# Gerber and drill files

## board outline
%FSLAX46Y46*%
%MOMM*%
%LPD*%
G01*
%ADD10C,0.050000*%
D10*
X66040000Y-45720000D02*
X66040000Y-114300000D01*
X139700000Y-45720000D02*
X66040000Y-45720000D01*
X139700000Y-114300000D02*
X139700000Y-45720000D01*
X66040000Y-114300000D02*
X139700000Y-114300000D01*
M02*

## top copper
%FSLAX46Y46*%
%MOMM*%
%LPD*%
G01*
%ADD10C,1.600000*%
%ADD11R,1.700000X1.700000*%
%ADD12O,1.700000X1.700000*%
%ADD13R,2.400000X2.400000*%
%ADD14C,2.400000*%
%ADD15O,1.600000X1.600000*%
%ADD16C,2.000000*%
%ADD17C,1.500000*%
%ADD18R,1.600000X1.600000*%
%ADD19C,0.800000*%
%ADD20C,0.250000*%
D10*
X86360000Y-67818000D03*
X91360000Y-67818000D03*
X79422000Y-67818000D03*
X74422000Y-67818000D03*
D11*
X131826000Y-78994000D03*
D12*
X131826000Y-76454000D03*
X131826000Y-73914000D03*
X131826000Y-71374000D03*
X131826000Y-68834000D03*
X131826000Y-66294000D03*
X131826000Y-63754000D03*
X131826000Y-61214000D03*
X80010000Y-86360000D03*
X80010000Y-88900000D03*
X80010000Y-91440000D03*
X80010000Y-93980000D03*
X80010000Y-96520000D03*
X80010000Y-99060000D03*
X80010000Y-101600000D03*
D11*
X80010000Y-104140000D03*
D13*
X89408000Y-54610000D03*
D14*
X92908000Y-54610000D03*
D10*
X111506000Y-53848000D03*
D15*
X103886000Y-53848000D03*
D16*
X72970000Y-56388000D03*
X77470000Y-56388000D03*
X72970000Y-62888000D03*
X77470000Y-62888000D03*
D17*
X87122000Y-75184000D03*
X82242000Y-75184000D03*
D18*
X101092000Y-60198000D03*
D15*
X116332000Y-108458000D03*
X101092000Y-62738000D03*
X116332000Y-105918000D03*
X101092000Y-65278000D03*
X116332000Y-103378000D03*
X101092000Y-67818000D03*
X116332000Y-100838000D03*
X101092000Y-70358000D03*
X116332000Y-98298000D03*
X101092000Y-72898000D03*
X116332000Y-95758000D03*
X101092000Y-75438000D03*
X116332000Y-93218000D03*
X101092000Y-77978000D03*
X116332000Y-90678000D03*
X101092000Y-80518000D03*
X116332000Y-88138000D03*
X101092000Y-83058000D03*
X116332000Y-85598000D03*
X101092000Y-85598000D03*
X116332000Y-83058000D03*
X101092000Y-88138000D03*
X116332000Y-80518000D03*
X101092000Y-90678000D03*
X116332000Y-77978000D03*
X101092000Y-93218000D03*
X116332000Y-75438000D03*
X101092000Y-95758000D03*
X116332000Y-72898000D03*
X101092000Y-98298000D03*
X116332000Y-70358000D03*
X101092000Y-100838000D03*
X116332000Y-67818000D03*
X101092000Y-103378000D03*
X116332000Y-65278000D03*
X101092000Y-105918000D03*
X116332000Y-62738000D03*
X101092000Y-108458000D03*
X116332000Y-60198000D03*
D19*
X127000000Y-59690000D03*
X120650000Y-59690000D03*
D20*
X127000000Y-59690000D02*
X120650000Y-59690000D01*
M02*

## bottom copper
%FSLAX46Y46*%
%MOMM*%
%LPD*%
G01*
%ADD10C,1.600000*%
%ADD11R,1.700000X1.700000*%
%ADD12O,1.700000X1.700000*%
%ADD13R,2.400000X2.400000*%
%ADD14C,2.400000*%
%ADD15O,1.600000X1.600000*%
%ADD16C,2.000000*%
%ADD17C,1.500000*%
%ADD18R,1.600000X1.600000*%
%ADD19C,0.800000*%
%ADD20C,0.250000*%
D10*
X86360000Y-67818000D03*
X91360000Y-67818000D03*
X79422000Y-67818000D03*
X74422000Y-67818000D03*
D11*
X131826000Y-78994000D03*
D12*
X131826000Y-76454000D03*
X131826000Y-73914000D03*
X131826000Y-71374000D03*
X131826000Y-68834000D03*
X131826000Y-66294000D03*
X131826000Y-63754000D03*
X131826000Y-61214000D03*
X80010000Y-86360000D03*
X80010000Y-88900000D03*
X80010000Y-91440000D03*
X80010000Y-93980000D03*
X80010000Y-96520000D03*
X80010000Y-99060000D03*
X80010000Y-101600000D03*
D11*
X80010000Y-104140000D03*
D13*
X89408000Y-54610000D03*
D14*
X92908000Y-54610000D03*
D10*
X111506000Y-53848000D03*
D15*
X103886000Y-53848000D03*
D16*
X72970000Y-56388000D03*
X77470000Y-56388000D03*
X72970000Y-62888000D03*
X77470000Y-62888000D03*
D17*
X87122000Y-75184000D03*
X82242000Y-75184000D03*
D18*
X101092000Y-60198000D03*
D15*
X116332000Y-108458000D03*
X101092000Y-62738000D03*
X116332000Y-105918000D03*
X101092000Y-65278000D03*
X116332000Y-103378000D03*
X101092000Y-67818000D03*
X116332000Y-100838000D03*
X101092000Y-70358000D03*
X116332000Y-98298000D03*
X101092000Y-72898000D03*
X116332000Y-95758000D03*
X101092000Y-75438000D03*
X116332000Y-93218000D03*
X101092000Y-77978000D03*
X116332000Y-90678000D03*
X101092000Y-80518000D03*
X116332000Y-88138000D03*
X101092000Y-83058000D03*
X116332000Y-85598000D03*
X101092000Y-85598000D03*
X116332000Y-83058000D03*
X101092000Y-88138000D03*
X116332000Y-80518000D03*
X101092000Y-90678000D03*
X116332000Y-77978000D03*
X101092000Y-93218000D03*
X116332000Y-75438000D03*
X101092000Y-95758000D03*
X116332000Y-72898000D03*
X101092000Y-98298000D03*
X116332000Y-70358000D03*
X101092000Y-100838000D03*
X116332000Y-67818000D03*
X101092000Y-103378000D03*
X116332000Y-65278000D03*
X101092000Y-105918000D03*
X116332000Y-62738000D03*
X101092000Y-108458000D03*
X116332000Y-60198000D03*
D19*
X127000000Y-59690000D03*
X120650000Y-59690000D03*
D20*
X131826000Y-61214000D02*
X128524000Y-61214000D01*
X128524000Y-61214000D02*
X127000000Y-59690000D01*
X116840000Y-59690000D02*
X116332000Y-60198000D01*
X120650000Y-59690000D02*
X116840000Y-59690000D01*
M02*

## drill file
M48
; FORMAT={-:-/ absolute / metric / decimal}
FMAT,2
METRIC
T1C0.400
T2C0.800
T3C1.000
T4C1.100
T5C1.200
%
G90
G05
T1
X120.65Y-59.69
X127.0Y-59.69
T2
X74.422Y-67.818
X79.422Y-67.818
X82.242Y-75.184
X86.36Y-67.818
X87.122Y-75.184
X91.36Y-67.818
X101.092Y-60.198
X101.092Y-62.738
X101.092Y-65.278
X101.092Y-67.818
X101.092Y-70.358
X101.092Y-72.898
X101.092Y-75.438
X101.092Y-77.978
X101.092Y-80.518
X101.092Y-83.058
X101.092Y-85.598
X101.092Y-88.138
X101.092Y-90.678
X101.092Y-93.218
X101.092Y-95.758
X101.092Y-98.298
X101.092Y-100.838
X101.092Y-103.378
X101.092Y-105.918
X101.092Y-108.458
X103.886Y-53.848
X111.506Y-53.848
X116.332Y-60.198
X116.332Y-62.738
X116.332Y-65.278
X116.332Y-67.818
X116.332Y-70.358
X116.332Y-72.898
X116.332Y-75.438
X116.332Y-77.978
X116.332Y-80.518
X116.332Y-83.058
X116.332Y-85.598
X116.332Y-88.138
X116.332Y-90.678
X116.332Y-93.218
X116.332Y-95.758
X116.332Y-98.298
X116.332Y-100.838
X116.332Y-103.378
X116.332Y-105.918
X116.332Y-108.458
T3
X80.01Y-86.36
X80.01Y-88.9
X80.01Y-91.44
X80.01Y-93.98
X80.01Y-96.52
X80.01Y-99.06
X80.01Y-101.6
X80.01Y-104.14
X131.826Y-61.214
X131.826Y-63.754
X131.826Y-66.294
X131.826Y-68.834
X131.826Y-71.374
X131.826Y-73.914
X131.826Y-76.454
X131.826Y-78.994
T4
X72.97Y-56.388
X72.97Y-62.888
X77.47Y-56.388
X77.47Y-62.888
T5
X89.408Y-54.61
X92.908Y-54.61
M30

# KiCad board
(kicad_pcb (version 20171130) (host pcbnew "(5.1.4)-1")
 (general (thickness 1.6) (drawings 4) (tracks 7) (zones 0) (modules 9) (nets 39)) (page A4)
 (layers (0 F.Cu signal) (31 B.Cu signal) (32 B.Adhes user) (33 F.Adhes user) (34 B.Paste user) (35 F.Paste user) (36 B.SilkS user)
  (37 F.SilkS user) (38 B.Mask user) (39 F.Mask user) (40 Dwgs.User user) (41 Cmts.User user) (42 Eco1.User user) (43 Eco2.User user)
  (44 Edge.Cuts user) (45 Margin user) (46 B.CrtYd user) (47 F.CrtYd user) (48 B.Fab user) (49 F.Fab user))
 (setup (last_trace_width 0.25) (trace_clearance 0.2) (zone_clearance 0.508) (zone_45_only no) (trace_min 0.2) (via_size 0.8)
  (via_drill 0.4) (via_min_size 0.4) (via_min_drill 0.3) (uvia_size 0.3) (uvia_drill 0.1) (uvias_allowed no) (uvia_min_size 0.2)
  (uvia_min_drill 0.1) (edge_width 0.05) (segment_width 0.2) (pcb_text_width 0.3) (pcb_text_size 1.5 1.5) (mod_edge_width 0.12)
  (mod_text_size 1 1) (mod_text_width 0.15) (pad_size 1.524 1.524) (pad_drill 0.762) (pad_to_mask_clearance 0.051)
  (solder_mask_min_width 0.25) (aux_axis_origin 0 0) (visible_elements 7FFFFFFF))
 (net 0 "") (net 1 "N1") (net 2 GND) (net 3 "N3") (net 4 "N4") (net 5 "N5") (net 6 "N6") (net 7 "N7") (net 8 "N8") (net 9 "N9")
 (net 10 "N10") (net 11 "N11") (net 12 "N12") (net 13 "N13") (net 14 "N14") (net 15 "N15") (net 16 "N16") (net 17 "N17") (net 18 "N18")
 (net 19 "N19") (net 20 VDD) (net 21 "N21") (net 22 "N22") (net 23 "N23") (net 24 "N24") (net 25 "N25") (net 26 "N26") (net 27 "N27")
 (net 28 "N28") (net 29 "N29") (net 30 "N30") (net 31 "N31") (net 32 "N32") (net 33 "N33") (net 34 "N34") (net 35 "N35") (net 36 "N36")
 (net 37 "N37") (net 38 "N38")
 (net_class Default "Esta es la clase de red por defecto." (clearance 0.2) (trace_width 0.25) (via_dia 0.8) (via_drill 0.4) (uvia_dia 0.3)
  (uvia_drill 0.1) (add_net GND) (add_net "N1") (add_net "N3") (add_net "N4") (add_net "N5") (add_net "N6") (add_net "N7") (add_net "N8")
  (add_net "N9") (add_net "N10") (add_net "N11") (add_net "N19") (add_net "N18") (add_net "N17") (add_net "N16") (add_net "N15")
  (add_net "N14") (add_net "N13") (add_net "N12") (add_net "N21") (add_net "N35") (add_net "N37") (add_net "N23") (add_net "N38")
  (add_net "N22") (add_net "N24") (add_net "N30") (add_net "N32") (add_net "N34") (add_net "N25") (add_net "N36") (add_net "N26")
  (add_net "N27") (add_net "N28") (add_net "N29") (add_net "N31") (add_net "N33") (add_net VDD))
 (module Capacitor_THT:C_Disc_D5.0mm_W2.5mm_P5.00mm (layer F.Cu) (at 86.36 67.818)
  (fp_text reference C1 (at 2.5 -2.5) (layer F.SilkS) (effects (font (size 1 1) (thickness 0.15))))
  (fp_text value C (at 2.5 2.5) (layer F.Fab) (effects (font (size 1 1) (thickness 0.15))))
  (pad 1 thru_hole circle (at 0 0) (size 1.6 1.6) (drill 0.8) (layers *.Cu *.Mask) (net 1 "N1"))
  (pad 2 thru_hole circle (at 5 0) (size 1.6 1.6) (drill 0.8) (layers *.Cu *.Mask) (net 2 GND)))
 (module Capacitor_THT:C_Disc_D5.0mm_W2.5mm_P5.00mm (layer F.Cu) (at 74.422 67.818)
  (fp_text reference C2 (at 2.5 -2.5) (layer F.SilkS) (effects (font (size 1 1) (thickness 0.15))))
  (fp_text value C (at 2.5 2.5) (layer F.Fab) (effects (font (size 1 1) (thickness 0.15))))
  (pad 2 thru_hole circle (at 5 0) (size 1.6 1.6) (drill 0.8) (layers *.Cu *.Mask) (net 2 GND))
  (pad 1 thru_hole circle (at 0 0) (size 1.6 1.6) (drill 0.8) (layers *.Cu *.Mask) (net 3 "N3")))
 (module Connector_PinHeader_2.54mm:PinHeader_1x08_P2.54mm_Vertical (layer F.Cu) (at 131.826 78.994 180)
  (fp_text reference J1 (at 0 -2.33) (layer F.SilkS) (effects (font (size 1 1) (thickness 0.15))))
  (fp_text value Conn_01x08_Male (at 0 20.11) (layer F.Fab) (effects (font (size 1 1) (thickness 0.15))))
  (pad 1 thru_hole rect (at 0 0 180) (size 1.7 1.7) (drill 1) (layers *.Cu *.Mask) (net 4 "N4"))
  (pad 2 thru_hole oval (at 0 2.54 180) (size 1.7 1.7) (drill 1) (layers *.Cu *.Mask) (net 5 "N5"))
  (pad 3 thru_hole oval (at 0 5.08 180) (size 1.7 1.7) (drill 1) (layers *.Cu *.Mask) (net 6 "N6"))
  (pad 4 thru_hole oval (at 0 7.62 180) (size 1.7 1.7) (drill 1) (layers *.Cu *.Mask) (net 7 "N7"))
  (pad 5 thru_hole oval (at 0 10.16 180) (size 1.7 1.7) (drill 1) (layers *.Cu *.Mask) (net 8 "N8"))
  (pad 6 thru_hole oval (at 0 12.7 180) (size 1.7 1.7) (drill 1) (layers *.Cu *.Mask) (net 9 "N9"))
  (pad 7 thru_hole oval (at 0 15.24 180) (size 1.7 1.7) (drill 1) (layers *.Cu *.Mask) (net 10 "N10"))
  (pad 8 thru_hole oval (at 0 17.78 180) (size 1.7 1.7) (drill 1) (layers *.Cu *.Mask) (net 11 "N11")))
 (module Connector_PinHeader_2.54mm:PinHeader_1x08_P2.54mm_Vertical (layer F.Cu) (at 80.01 104.14 180)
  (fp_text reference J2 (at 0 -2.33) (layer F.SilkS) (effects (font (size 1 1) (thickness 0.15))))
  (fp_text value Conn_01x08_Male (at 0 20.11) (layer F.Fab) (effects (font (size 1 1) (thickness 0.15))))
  (pad 8 thru_hole oval (at 0 17.78 180) (size 1.7 1.7) (drill 1) (layers *.Cu *.Mask) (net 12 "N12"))
  (pad 7 thru_hole oval (at 0 15.24 180) (size 1.7 1.7) (drill 1) (layers *.Cu *.Mask) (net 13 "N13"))
  (pad 6 thru_hole oval (at 0 12.7 180) (size 1.7 1.7) (drill 1) (layers *.Cu *.Mask) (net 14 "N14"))
  (pad 5 thru_hole oval (at 0 10.16 180) (size 1.7 1.7) (drill 1) (layers *.Cu *.Mask) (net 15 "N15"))
  (pad 4 thru_hole oval (at 0 7.62 180) (size 1.7 1.7) (drill 1) (layers *.Cu *.Mask) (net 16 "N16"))
  (pad 3 thru_hole oval (at 0 5.08 180) (size 1.7 1.7) (drill 1) (layers *.Cu *.Mask) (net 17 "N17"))
  (pad 2 thru_hole oval (at 0 2.54 180) (size 1.7 1.7) (drill 1) (layers *.Cu *.Mask) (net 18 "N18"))
  (pad 1 thru_hole rect (at 0 0 180) (size 1.7 1.7) (drill 1) (layers *.Cu *.Mask) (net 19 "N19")))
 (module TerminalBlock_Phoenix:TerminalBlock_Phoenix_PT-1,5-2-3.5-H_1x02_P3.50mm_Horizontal (layer F.Cu) (at 89.408 54.61)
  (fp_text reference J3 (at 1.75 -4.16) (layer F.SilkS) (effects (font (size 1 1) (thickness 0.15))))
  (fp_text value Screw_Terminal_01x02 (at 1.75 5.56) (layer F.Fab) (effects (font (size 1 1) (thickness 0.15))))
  (pad 1 thru_hole rect (at 0 0) (size 2.4 2.4) (drill 1.2) (layers *.Cu *.Mask) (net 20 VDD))
  (pad 2 thru_hole circle (at 3.5 0) (size 2.4 2.4) (drill 1.2) (layers *.Cu *.Mask) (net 2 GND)))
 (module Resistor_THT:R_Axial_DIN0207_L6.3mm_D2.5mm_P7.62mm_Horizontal (layer F.Cu) (at 111.506 53.848 180)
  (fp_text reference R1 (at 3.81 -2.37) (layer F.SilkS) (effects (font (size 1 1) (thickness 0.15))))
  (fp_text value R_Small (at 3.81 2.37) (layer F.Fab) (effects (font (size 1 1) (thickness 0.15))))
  (pad 1 thru_hole circle (at 0 0 180) (size 1.6 1.6) (drill 0.8) (layers *.Cu *.Mask) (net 20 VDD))
  (pad 2 thru_hole oval (at 7.62 0 180) (size 1.6 1.6) (drill 0.8) (layers *.Cu *.Mask) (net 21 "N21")))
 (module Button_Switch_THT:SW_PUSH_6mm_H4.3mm (layer F.Cu) (at 77.47 56.388 270)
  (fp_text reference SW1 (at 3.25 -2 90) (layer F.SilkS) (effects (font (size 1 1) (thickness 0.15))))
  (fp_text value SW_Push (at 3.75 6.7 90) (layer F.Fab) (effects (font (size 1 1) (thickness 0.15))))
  (pad 2 thru_hole circle (at 0 4.5) (size 2 2) (drill 1.1) (layers *.Cu *.Mask) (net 21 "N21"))
  (pad 1 thru_hole circle (at 0 0) (size 2 2) (drill 1.1) (layers *.Cu *.Mask) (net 2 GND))
  (pad 2 thru_hole circle (at 6.5 4.5) (size 2 2) (drill 1.1) (layers *.Cu *.Mask) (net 21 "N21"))
  (pad 1 thru_hole circle (at 6.5 0) (size 2 2) (drill 1.1) (layers *.Cu *.Mask) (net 2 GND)))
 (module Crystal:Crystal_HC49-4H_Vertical (layer F.Cu) (at 87.122 75.184 180)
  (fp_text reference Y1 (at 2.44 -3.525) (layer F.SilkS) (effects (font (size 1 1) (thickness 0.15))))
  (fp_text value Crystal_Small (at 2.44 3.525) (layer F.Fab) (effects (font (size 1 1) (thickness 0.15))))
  (pad 1 thru_hole circle (at 0 0 180) (size 1.5 1.5) (drill 0.8) (layers *.Cu *.Mask) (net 1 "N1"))
  (pad 2 thru_hole circle (at 4.88 0 180) (size 1.5 1.5) (drill 0.8) (layers *.Cu *.Mask) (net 3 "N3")))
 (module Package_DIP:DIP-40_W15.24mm (layer F.Cu) (at 101.092 60.198)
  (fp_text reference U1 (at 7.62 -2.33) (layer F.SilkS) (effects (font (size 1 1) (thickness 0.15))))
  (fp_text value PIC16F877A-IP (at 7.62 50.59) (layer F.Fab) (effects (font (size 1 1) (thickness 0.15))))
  (pad 1 thru_hole rect (at 0 0) (size 1.6 1.6) (drill 0.8) (layers *.Cu *.Mask) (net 21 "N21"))
  (pad 21 thru_hole oval (at 15.24 48.26) (size 1.6 1.6) (drill 0.8) (layers *.Cu *.Mask) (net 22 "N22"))
  (pad 2 thru_hole oval (at 0 2.54) (size 1.6 1.6) (drill 0.8) (layers *.Cu *.Mask) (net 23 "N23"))
  (pad 22 thru_hole oval (at 15.24 45.72) (size 1.6 1.6) (drill 0.8) (layers *.Cu *.Mask) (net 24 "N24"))
  (pad 3 thru_hole oval (at 0 5.08) (size 1.6 1.6) (drill 0.8) (layers *.Cu *.Mask) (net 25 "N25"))
  (pad 23 thru_hole oval (at 15.24 43.18) (size 1.6 1.6) (drill 0.8) (layers *.Cu *.Mask) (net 15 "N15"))
  (pad 4 thru_hole oval (at 0 7.62) (size 1.6 1.6) (drill 0.8) (layers *.Cu *.Mask) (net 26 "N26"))
  (pad 24 thru_hole oval (at 15.24 40.64) (size 1.6 1.6) (drill 0.8) (layers *.Cu *.Mask) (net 14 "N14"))
  (pad 5 thru_hole oval (at 0 10.16) (size 1.6 1.6) (drill 0.8) (layers *.Cu *.Mask) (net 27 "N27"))
  (pad 25 thru_hole oval (at 15.24 38.1) (size 1.6 1.6) (drill 0.8) (layers *.Cu *.Mask) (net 13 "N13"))
  (pad 6 thru_hole oval (at 0 12.7) (size 1.6 1.6) (drill 0.8) (layers *.Cu *.Mask) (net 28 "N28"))
  (pad 26 thru_hole oval (at 15.24 35.56) (size 1.6 1.6) (drill 0.8) (layers *.Cu *.Mask) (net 12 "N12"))
  (pad 7 thru_hole oval (at 0 15.24) (size 1.6 1.6) (drill 0.8) (layers *.Cu *.Mask) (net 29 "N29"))
  (pad 27 thru_hole oval (at 15.24 33.02) (size 1.6 1.6) (drill 0.8) (layers *.Cu *.Mask) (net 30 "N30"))
  (pad 8 thru_hole oval (at 0 17.78) (size 1.6 1.6) (drill 0.8) (layers *.Cu *.Mask) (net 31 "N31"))
  (pad 28 thru_hole oval (at 15.24 30.48) (size 1.6 1.6) (drill 0.8) (layers *.Cu *.Mask) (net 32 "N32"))
  (pad 9 thru_hole oval (at 0 20.32) (size 1.6 1.6) (drill 0.8) (layers *.Cu *.Mask) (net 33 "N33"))
  (pad 29 thru_hole oval (at 15.24 27.94) (size 1.6 1.6) (drill 0.8) (layers *.Cu *.Mask) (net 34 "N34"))
  (pad 10 thru_hole oval (at 0 22.86) (size 1.6 1.6) (drill 0.8) (layers *.Cu *.Mask) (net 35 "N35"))
  (pad 30 thru_hole oval (at 15.24 25.4) (size 1.6 1.6) (drill 0.8) (layers *.Cu *.Mask) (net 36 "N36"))
  (pad 11 thru_hole oval (at 0 25.4) (size 1.6 1.6) (drill 0.8) (layers *.Cu *.Mask) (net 20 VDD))
  (pad 31 thru_hole oval (at 15.24 22.86) (size 1.6 1.6) (drill 0.8) (layers *.Cu *.Mask) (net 2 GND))
  (pad 12 thru_hole oval (at 0 27.94) (size 1.6 1.6) (drill 0.8) (layers *.Cu *.Mask) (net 2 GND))
  (pad 32 thru_hole oval (at 15.24 20.32) (size 1.6 1.6) (drill 0.8) (layers *.Cu *.Mask) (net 20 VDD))
  (pad 13 thru_hole oval (at 0 30.48) (size 1.6 1.6) (drill 0.8) (layers *.Cu *.Mask) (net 1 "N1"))
  (pad 33 thru_hole oval (at 15.24 17.78) (size 1.6 1.6) (drill 0.8) (layers *.Cu *.Mask) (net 4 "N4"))
  (pad 14 thru_hole oval (at 0 33.02) (size 1.6 1.6) (drill 0.8) (layers *.Cu *.Mask) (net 3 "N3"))
  (pad 34 thru_hole oval (at 15.24 15.24) (size 1.6 1.6) (drill 0.8) (layers *.Cu *.Mask) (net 5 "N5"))
  (pad 15 thru_hole oval (at 0 35.56) (size 1.6 1.6) (drill 0.8) (layers *.Cu *.Mask) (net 19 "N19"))
  (pad 35 thru_hole oval (at 15.24 12.7) (size 1.6 1.6) (drill 0.8) (layers *.Cu *.Mask) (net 6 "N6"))
  (pad 16 thru_hole oval (at 0 38.1) (size 1.6 1.6) (drill 0.8) (layers *.Cu *.Mask) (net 18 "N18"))
  (pad 36 thru_hole oval (at 15.24 10.16) (size 1.6 1.6) (drill 0.8) (layers *.Cu *.Mask) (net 7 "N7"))
  (pad 17 thru_hole oval (at 0 40.64) (size 1.6 1.6) (drill 0.8) (layers *.Cu *.Mask) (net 17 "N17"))
  (pad 37 thru_hole oval (at 15.24 7.62) (size 1.6 1.6) (drill 0.8) (layers *.Cu *.Mask) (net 8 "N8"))
  (pad 18 thru_hole oval (at 0 43.18) (size 1.6 1.6) (drill 0.8) (layers *.Cu *.Mask) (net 16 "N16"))
  (pad 38 thru_hole oval (at 15.24 5.08) (size 1.6 1.6) (drill 0.8) (layers *.Cu *.Mask) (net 9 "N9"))
  (pad 19 thru_hole oval (at 0 45.72) (size 1.6 1.6) (drill 0.8) (layers *.Cu *.Mask) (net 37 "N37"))
  (pad 39 thru_hole oval (at 15.24 2.54) (size 1.6 1.6) (drill 0.8) (layers *.Cu *.Mask) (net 10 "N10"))
  (pad 20 thru_hole oval (at 0 48.26) (size 1.6 1.6) (drill 0.8) (layers *.Cu *.Mask) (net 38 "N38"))
  (pad 40 thru_hole oval (at 15.24 0) (size 1.6 1.6) (drill 0.8) (layers *.Cu *.Mask) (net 11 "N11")))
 (gr_line (start 66.04 45.72) (end 66.04 114.3) (layer Edge.Cuts) (width 0.05))
 (gr_line (start 139.7 45.72) (end 66.04 45.72) (layer Edge.Cuts) (width 0.05))
 (gr_line (start 139.7 114.3) (end 139.7 45.72) (layer Edge.Cuts) (width 0.05))
 (gr_line (start 66.04 114.3) (end 139.7 114.3) (layer Edge.Cuts) (width 0.05))
 (via (at 127 59.69) (size 0.8) (drill 0.4) (layers F.Cu B.Cu) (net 11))
 (segment (start 131.826 61.214) (end 128.524 61.214) (width 0.25) (layer B.Cu) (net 11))
 (segment (start 128.524 61.214) (end 127 59.69) (width 0.25) (layer B.Cu) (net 11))
 (via (at 120.65 59.69) (size 0.8) (drill 0.4) (layers F.Cu B.Cu) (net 11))
 (segment (start 127 59.69) (end 120.65 59.69) (width 0.25) (layer F.Cu) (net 11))
 (segment (start 116.84 59.69) (end 116.332 60.198) (width 0.25) (layer B.Cu) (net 11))
 (segment (start 120.65 59.69) (end 116.84 59.69) (width 0.25) (layer B.Cu) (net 11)))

